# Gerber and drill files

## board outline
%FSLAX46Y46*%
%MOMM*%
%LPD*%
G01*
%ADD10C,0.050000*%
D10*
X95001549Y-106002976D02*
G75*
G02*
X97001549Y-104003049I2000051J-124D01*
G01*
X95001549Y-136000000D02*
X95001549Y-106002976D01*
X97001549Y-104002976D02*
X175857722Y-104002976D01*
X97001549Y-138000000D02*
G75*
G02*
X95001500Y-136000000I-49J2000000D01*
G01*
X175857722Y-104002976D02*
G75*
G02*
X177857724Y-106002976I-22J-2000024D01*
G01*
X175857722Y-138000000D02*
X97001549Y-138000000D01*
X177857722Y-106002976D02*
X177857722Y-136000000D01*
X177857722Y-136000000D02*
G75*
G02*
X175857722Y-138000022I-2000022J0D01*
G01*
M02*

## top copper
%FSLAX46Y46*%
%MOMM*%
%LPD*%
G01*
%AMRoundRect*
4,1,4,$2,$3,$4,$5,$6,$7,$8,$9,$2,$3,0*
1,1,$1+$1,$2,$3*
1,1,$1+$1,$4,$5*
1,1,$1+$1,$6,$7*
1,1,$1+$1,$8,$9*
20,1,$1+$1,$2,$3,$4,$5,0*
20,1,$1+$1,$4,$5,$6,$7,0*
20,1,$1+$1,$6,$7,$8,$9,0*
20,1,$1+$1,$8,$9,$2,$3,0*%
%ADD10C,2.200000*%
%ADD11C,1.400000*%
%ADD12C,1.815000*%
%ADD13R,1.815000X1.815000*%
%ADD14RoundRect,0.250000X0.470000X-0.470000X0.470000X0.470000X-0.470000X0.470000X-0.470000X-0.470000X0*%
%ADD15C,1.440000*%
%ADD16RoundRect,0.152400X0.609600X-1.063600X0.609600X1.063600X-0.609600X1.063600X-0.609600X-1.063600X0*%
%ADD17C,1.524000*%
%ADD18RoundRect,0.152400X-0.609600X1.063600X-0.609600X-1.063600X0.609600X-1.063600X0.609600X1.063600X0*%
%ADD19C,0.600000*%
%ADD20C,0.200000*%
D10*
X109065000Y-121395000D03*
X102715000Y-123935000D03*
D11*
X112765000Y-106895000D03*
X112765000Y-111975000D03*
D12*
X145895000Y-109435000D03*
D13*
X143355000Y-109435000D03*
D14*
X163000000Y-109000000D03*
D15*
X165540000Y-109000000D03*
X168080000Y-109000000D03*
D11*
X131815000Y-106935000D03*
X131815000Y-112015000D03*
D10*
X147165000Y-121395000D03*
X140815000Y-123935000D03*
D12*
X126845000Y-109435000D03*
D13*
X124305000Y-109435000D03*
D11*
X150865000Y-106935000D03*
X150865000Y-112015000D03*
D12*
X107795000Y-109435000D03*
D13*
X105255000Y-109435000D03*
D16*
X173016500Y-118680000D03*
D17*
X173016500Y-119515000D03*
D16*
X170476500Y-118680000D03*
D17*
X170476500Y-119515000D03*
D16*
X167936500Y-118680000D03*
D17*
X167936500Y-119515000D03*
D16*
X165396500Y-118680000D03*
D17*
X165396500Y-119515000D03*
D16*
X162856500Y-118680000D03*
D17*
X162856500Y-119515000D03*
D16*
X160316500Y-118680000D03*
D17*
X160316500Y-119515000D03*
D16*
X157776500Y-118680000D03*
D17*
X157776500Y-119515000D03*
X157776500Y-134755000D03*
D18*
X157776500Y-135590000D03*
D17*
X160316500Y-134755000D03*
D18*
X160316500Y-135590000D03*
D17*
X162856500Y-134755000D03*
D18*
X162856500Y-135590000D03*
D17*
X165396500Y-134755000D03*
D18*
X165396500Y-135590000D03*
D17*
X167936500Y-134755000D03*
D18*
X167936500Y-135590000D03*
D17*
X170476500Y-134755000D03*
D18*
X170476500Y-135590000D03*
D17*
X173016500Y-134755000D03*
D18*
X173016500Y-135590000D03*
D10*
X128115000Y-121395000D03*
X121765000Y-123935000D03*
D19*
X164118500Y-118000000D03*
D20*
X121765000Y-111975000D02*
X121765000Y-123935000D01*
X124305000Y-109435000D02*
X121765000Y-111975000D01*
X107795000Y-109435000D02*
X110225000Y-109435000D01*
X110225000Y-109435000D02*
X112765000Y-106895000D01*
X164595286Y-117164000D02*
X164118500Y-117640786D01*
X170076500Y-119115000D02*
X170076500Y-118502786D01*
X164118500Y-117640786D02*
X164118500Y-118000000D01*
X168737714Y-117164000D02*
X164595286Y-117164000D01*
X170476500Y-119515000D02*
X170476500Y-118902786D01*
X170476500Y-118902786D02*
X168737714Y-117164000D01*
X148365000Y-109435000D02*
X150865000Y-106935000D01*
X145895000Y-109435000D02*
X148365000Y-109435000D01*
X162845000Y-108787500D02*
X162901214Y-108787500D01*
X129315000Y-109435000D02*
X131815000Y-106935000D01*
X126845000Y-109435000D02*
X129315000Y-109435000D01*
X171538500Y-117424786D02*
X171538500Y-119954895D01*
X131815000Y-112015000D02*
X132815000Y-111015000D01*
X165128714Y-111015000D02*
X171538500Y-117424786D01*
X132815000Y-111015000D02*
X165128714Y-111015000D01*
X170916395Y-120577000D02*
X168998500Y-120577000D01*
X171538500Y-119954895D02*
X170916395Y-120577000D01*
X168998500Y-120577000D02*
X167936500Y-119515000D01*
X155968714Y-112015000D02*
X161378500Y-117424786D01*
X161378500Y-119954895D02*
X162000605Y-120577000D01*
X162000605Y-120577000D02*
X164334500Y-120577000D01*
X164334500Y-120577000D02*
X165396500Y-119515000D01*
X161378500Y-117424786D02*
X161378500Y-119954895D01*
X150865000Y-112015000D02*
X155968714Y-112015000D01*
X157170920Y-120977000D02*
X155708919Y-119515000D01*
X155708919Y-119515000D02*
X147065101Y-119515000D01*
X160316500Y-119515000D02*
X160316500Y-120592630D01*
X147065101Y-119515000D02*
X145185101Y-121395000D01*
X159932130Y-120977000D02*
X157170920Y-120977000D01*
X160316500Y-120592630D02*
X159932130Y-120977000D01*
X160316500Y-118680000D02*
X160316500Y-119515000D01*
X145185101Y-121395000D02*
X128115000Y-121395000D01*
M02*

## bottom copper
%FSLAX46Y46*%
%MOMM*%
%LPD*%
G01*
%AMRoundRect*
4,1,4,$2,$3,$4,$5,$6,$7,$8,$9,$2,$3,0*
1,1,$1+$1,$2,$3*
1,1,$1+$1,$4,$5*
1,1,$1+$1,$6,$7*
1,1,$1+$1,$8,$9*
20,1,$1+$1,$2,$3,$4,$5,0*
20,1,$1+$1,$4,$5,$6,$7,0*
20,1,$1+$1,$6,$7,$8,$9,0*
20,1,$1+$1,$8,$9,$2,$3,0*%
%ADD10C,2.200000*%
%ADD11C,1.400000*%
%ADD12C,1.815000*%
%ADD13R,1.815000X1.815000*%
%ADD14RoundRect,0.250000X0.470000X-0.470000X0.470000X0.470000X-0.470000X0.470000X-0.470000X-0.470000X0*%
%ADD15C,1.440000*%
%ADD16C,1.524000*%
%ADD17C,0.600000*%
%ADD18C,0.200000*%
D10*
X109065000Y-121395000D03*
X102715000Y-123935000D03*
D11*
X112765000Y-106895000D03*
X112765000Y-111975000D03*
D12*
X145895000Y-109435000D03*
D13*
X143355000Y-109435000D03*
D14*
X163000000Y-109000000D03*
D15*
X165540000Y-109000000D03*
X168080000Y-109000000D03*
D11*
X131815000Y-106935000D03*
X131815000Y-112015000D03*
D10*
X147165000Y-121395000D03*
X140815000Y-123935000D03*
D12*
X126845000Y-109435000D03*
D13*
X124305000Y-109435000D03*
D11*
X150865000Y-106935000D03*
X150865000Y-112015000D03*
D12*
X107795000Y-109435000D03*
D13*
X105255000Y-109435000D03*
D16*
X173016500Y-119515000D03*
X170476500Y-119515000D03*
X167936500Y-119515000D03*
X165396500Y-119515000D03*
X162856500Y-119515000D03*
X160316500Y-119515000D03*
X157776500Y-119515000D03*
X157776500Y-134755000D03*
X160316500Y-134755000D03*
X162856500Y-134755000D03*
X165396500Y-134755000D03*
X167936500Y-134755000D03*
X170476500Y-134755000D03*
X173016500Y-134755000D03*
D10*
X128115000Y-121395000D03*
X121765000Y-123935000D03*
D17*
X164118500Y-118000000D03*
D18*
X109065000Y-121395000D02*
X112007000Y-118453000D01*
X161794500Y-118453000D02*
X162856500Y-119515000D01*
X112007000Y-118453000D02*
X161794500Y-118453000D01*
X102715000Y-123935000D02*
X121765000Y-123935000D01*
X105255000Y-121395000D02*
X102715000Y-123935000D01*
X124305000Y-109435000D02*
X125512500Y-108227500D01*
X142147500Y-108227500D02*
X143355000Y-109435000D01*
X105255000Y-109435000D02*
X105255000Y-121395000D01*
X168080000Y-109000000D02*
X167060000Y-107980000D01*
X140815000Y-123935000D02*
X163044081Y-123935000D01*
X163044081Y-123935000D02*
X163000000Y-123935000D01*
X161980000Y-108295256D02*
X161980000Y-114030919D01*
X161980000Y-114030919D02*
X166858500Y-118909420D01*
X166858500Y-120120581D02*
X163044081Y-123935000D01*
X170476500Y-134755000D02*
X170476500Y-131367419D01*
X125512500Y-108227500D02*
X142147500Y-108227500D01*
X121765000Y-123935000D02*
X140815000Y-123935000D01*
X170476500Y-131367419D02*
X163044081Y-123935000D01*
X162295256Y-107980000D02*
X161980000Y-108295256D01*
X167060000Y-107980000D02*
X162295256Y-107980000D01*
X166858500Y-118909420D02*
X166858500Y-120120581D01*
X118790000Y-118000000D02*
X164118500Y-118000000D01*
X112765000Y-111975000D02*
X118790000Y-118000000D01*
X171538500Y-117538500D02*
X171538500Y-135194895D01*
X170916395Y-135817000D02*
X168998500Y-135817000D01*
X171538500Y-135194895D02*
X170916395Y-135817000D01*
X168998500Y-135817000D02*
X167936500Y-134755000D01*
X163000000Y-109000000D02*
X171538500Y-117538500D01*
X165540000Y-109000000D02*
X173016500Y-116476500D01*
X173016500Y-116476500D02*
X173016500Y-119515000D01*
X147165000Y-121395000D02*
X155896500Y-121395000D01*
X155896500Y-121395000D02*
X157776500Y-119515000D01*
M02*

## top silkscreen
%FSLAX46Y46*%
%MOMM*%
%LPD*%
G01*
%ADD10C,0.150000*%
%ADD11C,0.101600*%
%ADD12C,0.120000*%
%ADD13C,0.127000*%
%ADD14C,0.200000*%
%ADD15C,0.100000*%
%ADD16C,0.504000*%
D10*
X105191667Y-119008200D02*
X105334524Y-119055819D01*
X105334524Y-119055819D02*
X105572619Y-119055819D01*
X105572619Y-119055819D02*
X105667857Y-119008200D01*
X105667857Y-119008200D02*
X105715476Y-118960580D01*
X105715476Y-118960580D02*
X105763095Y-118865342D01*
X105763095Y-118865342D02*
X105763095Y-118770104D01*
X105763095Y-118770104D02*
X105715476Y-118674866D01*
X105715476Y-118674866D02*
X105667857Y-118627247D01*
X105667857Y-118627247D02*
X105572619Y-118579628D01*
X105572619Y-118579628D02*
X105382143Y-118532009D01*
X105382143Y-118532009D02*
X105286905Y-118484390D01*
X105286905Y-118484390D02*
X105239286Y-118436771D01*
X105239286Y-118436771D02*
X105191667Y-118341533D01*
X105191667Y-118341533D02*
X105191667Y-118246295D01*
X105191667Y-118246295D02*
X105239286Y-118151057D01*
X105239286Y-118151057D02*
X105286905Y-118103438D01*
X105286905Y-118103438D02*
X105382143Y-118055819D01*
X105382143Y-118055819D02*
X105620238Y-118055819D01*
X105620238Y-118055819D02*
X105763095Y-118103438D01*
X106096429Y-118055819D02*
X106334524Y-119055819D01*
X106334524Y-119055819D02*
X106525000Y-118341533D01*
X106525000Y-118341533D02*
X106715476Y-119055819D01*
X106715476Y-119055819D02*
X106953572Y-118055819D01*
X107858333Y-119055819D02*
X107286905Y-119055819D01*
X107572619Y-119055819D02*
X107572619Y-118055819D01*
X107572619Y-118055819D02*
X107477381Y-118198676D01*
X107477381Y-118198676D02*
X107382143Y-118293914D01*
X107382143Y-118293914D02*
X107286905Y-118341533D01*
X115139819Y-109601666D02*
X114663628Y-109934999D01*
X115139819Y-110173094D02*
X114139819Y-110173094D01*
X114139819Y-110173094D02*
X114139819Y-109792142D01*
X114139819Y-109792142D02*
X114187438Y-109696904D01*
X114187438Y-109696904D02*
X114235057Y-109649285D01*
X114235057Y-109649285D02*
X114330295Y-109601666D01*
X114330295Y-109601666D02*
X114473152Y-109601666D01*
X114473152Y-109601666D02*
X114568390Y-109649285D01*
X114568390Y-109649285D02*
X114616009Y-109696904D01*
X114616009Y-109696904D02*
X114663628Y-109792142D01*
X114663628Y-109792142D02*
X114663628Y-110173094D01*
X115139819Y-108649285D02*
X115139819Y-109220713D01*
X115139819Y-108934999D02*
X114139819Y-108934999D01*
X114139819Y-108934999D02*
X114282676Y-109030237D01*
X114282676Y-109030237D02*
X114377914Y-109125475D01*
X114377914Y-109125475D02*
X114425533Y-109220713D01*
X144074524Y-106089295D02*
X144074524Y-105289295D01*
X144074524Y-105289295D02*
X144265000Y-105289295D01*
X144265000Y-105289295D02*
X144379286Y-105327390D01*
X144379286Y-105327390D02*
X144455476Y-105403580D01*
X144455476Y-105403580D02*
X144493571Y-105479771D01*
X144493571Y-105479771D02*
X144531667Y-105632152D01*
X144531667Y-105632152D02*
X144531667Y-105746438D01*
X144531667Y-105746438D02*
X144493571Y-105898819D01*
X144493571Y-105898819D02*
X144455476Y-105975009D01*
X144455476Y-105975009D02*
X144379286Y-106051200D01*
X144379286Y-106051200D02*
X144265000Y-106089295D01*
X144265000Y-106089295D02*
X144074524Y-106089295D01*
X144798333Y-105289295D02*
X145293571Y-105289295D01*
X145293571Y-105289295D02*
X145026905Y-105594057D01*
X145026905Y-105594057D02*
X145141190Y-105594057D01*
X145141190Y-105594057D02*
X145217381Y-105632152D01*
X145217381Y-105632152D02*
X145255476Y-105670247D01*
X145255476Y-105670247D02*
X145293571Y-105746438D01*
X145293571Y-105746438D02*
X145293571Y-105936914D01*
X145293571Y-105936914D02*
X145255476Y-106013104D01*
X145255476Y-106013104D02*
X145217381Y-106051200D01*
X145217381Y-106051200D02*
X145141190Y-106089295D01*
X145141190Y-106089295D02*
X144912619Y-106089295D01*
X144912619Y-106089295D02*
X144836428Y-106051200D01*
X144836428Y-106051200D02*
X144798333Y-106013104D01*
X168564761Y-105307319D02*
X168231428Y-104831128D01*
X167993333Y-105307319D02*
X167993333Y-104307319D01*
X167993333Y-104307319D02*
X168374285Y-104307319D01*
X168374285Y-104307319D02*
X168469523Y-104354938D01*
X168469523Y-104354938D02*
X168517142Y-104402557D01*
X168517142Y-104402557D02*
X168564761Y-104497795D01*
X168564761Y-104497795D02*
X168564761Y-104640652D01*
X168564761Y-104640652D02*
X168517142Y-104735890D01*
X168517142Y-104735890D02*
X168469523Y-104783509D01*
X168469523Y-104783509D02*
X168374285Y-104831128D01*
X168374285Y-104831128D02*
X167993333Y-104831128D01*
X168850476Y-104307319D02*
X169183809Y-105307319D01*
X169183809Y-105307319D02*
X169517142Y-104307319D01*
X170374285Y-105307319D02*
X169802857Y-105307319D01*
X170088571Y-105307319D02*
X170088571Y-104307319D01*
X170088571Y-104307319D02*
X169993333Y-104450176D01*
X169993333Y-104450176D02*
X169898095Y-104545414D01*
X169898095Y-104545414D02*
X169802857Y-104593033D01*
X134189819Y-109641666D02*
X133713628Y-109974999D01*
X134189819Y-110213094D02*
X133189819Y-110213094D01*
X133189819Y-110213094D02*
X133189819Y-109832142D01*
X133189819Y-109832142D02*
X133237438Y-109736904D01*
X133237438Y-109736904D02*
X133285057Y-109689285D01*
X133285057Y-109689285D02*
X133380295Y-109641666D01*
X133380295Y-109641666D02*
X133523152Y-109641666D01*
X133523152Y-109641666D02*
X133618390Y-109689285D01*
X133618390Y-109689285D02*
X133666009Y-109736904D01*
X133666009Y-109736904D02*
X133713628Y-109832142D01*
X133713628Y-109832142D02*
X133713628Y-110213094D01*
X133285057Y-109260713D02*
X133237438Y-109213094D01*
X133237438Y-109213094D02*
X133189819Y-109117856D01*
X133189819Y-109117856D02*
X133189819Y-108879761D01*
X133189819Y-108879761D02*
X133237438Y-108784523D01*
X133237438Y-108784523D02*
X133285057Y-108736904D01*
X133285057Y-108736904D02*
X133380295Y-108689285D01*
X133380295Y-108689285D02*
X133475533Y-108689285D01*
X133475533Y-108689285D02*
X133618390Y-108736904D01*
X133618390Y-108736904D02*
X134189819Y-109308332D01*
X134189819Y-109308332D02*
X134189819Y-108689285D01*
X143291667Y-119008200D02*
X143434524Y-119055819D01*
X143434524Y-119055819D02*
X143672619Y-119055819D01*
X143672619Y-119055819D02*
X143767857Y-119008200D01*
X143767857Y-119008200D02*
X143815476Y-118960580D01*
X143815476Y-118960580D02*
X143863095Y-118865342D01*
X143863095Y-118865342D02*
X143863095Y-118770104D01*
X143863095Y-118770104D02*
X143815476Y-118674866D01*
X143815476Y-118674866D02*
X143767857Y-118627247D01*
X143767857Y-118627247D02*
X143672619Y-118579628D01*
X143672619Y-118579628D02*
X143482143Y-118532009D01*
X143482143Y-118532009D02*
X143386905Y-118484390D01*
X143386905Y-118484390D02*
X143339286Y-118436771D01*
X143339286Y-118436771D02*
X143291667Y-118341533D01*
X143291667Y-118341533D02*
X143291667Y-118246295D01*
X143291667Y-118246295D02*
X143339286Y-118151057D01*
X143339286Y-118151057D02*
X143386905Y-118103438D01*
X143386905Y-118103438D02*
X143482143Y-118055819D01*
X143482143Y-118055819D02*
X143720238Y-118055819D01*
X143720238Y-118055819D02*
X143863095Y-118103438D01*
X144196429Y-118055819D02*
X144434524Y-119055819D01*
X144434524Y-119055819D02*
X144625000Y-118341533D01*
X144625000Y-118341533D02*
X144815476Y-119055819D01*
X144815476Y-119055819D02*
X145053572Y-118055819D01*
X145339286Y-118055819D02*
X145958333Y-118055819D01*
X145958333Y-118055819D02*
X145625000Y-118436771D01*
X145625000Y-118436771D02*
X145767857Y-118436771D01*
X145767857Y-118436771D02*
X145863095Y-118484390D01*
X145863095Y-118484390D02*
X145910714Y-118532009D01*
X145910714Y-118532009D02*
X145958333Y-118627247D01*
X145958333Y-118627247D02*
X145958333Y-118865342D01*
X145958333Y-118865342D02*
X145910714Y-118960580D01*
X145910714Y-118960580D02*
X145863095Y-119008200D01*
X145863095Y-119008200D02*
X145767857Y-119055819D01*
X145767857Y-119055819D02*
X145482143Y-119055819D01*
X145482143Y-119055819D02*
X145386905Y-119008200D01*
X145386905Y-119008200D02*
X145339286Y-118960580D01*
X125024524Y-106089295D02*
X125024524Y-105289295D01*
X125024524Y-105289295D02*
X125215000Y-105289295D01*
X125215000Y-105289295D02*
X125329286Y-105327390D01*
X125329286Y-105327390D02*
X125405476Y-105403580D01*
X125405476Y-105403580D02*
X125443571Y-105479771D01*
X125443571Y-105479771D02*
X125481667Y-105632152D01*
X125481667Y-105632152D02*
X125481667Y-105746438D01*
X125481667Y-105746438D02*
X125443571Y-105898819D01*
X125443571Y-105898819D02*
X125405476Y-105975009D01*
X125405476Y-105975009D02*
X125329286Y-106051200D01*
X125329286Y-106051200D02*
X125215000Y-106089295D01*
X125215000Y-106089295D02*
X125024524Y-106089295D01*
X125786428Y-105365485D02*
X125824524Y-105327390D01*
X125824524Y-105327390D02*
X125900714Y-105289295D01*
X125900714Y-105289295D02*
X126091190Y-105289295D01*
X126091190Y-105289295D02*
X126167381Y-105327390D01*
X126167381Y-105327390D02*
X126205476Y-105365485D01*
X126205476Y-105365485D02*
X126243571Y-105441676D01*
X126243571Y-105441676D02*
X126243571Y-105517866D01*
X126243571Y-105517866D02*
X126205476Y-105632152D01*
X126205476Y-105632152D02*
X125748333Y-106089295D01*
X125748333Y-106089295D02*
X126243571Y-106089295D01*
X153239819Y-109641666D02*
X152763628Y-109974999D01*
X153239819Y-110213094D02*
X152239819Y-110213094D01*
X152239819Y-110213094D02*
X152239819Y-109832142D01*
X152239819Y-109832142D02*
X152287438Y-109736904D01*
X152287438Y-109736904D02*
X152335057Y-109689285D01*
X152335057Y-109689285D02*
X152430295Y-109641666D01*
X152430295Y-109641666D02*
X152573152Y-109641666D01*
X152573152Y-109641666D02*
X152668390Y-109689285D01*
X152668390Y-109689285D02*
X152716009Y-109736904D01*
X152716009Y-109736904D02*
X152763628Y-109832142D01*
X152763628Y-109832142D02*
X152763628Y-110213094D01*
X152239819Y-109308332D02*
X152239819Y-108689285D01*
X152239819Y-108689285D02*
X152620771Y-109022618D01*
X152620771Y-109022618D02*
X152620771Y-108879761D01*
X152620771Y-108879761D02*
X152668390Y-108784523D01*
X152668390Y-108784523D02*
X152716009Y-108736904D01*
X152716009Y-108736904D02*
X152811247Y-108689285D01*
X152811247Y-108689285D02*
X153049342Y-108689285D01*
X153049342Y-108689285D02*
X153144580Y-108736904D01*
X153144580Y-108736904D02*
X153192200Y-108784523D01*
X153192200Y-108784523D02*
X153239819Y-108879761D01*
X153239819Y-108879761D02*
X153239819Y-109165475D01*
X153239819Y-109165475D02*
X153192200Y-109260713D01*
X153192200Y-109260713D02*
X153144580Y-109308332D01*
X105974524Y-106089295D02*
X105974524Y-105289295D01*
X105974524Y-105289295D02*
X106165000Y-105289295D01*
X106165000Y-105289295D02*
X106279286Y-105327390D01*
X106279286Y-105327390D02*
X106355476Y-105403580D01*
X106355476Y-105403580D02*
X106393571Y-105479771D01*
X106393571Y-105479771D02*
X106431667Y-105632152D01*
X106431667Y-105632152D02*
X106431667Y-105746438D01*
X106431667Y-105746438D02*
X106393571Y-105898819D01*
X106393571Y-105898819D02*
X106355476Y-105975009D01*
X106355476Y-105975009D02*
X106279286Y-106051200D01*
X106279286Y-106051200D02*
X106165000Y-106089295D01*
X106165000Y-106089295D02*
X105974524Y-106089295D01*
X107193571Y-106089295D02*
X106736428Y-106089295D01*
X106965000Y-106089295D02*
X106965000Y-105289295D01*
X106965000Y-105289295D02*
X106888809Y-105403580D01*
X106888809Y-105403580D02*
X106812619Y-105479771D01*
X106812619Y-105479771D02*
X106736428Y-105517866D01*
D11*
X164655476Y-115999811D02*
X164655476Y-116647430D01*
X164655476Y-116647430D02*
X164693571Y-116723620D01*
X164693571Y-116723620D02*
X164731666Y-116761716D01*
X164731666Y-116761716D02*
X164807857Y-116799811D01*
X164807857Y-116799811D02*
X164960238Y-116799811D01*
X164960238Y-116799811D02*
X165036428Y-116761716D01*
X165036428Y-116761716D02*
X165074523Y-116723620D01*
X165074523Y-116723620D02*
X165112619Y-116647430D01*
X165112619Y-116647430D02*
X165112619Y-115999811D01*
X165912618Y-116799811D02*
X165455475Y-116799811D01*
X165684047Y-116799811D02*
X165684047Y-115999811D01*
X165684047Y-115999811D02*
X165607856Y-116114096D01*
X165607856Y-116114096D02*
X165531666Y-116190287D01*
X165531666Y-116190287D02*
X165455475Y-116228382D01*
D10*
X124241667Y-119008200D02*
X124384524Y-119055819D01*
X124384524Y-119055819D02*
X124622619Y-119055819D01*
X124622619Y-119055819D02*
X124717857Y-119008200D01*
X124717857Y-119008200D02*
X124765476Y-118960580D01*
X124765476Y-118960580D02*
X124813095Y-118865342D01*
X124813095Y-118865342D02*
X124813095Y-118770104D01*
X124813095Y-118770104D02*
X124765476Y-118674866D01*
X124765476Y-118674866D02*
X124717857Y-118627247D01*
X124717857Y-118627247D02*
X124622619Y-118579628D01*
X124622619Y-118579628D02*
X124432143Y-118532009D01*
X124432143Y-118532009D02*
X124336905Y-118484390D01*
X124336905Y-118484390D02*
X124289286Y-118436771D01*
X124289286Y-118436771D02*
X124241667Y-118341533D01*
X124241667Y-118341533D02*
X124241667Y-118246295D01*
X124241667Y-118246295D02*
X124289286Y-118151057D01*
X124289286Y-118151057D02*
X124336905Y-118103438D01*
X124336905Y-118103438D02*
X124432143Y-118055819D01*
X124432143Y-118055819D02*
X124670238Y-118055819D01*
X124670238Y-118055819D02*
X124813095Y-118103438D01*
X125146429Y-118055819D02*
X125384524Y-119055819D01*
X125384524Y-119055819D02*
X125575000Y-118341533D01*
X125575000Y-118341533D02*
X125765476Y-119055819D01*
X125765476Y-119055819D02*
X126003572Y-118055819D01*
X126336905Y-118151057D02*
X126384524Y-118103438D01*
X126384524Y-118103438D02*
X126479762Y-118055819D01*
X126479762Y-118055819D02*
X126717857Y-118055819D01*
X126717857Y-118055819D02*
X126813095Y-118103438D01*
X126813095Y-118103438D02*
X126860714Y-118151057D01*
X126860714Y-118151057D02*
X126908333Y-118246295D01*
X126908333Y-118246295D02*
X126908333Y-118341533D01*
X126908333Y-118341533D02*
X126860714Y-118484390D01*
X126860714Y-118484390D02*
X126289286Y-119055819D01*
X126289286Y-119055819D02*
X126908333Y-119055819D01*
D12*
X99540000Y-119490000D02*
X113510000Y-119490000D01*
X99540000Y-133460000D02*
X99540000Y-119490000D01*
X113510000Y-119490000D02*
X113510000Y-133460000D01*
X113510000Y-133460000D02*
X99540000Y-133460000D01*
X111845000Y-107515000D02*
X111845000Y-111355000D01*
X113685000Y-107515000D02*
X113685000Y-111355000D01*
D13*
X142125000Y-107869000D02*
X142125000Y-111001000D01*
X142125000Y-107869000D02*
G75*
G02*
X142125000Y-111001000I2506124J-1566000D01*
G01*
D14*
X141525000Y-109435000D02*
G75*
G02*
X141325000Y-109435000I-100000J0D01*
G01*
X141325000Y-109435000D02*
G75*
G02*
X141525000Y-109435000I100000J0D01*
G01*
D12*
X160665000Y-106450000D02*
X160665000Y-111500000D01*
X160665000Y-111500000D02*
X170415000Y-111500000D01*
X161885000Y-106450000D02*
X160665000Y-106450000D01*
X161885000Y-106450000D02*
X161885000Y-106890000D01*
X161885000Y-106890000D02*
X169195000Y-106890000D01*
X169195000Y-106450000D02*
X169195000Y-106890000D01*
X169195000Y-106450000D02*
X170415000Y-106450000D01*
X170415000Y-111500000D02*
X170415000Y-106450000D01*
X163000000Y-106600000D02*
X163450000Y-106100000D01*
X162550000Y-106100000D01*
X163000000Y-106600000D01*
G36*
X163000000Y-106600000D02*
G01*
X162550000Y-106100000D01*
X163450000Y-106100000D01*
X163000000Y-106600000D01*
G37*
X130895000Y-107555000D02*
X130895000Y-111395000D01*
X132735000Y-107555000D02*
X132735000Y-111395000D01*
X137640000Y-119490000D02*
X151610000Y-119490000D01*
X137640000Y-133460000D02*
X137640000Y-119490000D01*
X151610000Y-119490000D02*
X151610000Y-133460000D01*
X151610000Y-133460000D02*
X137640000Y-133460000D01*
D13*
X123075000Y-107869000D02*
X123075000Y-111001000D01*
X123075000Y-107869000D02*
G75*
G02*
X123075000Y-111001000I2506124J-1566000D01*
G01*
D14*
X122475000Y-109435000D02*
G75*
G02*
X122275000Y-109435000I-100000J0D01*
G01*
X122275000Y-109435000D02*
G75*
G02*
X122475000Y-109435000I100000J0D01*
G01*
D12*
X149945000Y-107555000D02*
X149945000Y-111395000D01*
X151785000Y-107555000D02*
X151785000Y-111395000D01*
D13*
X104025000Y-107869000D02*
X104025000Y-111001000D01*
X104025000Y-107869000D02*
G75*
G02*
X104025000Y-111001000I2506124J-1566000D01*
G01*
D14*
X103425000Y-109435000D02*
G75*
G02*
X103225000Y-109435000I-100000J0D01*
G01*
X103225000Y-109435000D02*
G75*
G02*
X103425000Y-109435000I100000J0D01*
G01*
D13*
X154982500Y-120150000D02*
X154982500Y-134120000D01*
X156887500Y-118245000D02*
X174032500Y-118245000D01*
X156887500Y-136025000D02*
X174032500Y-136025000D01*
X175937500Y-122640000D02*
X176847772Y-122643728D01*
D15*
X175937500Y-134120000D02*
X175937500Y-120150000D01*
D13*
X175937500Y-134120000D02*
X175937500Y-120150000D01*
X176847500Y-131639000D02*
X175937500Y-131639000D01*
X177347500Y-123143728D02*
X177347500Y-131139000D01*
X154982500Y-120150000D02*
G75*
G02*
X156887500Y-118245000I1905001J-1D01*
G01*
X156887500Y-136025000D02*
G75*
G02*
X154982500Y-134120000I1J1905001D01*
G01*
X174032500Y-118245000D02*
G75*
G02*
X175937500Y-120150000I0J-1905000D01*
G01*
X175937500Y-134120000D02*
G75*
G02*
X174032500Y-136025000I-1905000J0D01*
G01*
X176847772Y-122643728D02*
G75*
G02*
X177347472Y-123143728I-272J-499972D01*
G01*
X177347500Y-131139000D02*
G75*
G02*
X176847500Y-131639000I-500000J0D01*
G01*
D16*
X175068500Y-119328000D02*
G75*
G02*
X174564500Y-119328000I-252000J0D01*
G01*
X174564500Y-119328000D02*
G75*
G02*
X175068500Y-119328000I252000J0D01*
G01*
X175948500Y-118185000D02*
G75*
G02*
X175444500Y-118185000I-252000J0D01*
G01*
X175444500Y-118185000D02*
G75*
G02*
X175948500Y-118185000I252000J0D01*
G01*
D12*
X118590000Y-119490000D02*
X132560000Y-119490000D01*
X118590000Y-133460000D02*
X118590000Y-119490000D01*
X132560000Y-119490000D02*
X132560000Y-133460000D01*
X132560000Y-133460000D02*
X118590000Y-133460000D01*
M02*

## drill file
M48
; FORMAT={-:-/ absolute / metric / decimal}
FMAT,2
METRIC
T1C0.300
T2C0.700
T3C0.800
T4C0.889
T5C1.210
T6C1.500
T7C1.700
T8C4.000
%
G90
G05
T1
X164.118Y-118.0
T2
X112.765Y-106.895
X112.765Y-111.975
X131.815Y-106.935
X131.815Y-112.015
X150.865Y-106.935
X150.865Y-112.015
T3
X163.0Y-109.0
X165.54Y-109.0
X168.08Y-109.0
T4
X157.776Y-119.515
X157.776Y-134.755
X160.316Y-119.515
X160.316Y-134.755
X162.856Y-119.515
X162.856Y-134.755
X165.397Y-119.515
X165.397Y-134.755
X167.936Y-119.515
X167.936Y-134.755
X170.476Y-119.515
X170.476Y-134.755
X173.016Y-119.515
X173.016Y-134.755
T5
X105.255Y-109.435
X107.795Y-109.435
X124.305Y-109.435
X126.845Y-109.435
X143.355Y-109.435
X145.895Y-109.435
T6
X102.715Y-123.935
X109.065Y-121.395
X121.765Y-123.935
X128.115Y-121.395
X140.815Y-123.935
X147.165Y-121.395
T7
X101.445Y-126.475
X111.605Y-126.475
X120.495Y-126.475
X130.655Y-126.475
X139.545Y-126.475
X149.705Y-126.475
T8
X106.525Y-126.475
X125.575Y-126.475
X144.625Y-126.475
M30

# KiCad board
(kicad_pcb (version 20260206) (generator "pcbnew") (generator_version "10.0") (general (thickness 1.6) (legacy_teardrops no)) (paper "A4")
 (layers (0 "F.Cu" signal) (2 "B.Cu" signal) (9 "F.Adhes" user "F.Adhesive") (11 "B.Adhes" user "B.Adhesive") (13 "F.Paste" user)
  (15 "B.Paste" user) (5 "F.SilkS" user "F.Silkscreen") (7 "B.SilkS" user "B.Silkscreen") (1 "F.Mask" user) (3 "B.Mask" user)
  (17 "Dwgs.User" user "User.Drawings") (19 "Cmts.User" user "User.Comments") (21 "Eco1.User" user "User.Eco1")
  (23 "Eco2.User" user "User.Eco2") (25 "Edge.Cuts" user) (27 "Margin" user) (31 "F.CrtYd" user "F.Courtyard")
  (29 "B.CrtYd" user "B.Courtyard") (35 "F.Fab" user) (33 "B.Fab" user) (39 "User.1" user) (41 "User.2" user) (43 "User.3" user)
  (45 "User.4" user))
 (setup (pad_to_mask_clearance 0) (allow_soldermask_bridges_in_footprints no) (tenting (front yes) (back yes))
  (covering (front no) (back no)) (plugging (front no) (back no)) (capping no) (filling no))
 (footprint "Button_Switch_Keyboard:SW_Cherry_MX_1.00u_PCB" (layer "F.Cu") (at 109.065 121.395)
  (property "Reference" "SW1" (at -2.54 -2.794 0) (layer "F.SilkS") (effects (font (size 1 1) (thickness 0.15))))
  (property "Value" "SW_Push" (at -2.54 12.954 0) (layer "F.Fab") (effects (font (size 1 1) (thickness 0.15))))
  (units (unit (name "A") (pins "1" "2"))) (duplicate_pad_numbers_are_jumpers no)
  (fp_line (start -9.525 -1.905) (end 4.445 -1.905) (stroke (width 0.12) (type solid)) (layer "F.SilkS"))
  (fp_line (start -9.525 12.065) (end -9.525 -1.905) (stroke (width 0.12) (type solid)) (layer "F.SilkS"))
  (fp_line (start 4.445 -1.905) (end 4.445 12.065) (stroke (width 0.12) (type solid)) (layer "F.SilkS"))
  (fp_line (start 4.445 12.065) (end -9.525 12.065) (stroke (width 0.12) (type solid)) (layer "F.SilkS"))
  (pad "" np_thru_hole circle (at -7.62 5.08) (size 1.7 1.7) (drill 1.7) (layers "*.Cu" "*.Mask"))
  (pad "" np_thru_hole circle (at -2.54 5.08) (size 4 4) (drill 4) (layers "*.Cu" "*.Mask"))
  (pad "" np_thru_hole circle (at 2.54 5.08) (size 1.7 1.7) (drill 1.7) (layers "*.Cu" "*.Mask"))
  (pad "1" thru_hole circle (at 0 0) (size 2.2 2.2) (drill 1.5) (layers "*.Cu" "*.Mask") (remove_unused_layers no) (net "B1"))
  (pad "2" thru_hole circle (at -6.35 2.54) (size 2.2 2.2) (drill 1.5) (layers "*.Cu" "*.Mask") (remove_unused_layers no) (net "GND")))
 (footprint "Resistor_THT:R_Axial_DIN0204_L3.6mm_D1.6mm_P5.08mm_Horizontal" (layer "F.Cu") (at 112.765 106.895 -90)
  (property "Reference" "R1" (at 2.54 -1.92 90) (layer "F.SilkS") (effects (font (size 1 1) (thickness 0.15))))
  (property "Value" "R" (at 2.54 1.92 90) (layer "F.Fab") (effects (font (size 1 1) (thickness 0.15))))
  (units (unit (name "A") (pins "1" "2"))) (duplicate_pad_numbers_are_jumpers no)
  (fp_line (start 0.62 0.92) (end 4.46 0.92) (stroke (width 0.12) (type solid)) (layer "F.SilkS"))
  (fp_line (start 0.62 -0.92) (end 4.46 -0.92) (stroke (width 0.12) (type solid)) (layer "F.SilkS"))
  (pad "1" thru_hole circle (at 0 0 270) (size 1.4 1.4) (drill 0.7) (layers "*.Cu" "*.Mask") (remove_unused_layers no) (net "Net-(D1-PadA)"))
  (pad "2" thru_hole circle (at 5.08 0 270) (size 1.4 1.4) (drill 0.7) (layers "*.Cu" "*.Mask") (remove_unused_layers no) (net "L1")))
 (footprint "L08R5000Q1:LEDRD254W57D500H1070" (layer "F.Cu") (at 144.625 109.435)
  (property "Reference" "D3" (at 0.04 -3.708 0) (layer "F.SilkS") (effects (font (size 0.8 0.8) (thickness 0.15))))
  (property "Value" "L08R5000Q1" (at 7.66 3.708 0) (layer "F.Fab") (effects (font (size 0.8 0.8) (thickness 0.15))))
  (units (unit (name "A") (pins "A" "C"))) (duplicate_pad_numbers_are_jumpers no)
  (fp_line (start -2.5 -1.566) (end -2.5 1.566) (stroke (width 0.127) (type solid)) (layer "F.SilkS"))
  (fp_arc (start -2.5 -1.566) (mid 2.961291 0) (end -2.5 1.566) (stroke (width 0.127) (type solid)) (layer "F.SilkS"))
  (fp_circle (center -3.2 0) (end -3.1 0) (stroke (width 0.2) (type solid)) (fill no) (layer "F.SilkS"))
  (pad "A" thru_hole circle (at 1.27 0) (size 1.815 1.815) (drill 1.21) (layers "*.Cu" "*.Mask") (remove_unused_layers no)
   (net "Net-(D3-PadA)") (solder_mask_margin 0.102))
  (pad "C" thru_hole rect (at -1.27 0) (size 1.815 1.815) (drill 1.21) (layers "*.Cu" "*.Mask") (remove_unused_layers no) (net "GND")
   (solder_mask_margin 0.102)))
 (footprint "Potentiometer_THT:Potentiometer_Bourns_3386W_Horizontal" (layer "F.Cu") (at 163 109)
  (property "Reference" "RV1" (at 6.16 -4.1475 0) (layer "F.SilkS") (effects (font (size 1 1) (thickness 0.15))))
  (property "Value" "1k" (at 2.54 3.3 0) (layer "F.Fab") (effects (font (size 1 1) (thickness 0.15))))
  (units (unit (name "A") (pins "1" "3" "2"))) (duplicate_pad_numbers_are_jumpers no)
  (fp_line (start -2.335 -2.55) (end -2.335 2.5) (stroke (width 0.12) (type default)) (layer "F.SilkS"))
  (fp_line (start -2.335 2.5) (end 7.415 2.5) (stroke (width 0.12) (type default)) (layer "F.SilkS"))
  (fp_line (start -1.115 -2.55) (end -2.335 -2.55) (stroke (width 0.12) (type default)) (layer "F.SilkS"))
  (fp_line (start -1.115 -2.55) (end -1.115 -2.11) (stroke (width 0.12) (type default)) (layer "F.SilkS"))
  (fp_line (start -1.115 -2.11) (end 6.195 -2.11) (stroke (width 0.12) (type default)) (layer "F.SilkS"))
  (fp_line (start 6.195 -2.55) (end 6.195 -2.11) (stroke (width 0.12) (type default)) (layer "F.SilkS"))
  (fp_line (start 6.195 -2.55) (end 7.415 -2.55) (stroke (width 0.12) (type default)) (layer "F.SilkS"))
  (fp_line (start 7.415 2.5) (end 7.415 -2.55) (stroke (width 0.12) (type default)) (layer "F.SilkS"))
  (fp_poly (pts (xy 0 -2.4) (xy 0.45 -2.9) (xy -0.45 -2.9)) (stroke (width 0.12) (type solid)) (fill yes) (layer "F.SilkS"))
  (pad "1" thru_hole roundrect (at 0 0 90) (size 1.44 1.44) (drill 0.8) (layers "*.Cu" "*.Mask") (remove_unused_layers no)
   (roundrect_rratio 0.1736111111) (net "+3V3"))
  (pad "2" thru_hole circle (at 2.54 0 90) (size 1.44 1.44) (drill 0.8) (layers "*.Cu" "*.Mask") (remove_unused_layers no) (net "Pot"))
  (pad "3" thru_hole circle (at 5.08 0 90) (size 1.44 1.44) (drill 0.8) (layers "*.Cu" "*.Mask") (remove_unused_layers no) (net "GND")))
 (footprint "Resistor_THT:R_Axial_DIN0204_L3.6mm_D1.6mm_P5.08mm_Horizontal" (layer "F.Cu") (at 131.815 106.935 -90)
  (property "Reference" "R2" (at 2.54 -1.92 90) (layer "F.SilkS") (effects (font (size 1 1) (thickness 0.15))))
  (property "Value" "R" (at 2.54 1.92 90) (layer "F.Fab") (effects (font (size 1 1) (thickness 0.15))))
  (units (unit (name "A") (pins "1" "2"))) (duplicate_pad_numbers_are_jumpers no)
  (fp_line (start 0.62 0.92) (end 4.46 0.92) (stroke (width 0.12) (type solid)) (layer "F.SilkS"))
  (fp_line (start 0.62 -0.92) (end 4.46 -0.92) (stroke (width 0.12) (type solid)) (layer "F.SilkS"))
  (pad "1" thru_hole circle (at 0 0 270) (size 1.4 1.4) (drill 0.7) (layers "*.Cu" "*.Mask") (remove_unused_layers no) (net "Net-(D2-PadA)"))
  (pad "2" thru_hole circle (at 5.08 0 270) (size 1.4 1.4) (drill 0.7) (layers "*.Cu" "*.Mask") (remove_unused_layers no) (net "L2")))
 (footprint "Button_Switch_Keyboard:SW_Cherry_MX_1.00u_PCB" (layer "F.Cu") (at 147.165 121.395)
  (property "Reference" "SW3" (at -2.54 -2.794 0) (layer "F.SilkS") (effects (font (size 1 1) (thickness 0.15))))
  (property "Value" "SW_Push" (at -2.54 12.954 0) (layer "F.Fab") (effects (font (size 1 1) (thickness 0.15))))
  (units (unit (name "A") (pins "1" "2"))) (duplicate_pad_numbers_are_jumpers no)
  (fp_line (start -9.525 -1.905) (end 4.445 -1.905) (stroke (width 0.12) (type solid)) (layer "F.SilkS"))
  (fp_line (start -9.525 12.065) (end -9.525 -1.905) (stroke (width 0.12) (type solid)) (layer "F.SilkS"))
  (fp_line (start 4.445 -1.905) (end 4.445 12.065) (stroke (width 0.12) (type solid)) (layer "F.SilkS"))
  (fp_line (start 4.445 12.065) (end -9.525 12.065) (stroke (width 0.12) (type solid)) (layer "F.SilkS"))
  (pad "" np_thru_hole circle (at -7.62 5.08) (size 1.7 1.7) (drill 1.7) (layers "*.Cu" "*.Mask"))
  (pad "" np_thru_hole circle (at -2.54 5.08) (size 4 4) (drill 4) (layers "*.Cu" "*.Mask"))
  (pad "" np_thru_hole circle (at 2.54 5.08) (size 1.7 1.7) (drill 1.7) (layers "*.Cu" "*.Mask"))
  (pad "1" thru_hole circle (at 0 0) (size 2.2 2.2) (drill 1.5) (layers "*.Cu" "*.Mask") (remove_unused_layers no) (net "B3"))
  (pad "2" thru_hole circle (at -6.35 2.54) (size 2.2 2.2) (drill 1.5) (layers "*.Cu" "*.Mask") (remove_unused_layers no) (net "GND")))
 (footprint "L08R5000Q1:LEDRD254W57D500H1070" (layer "F.Cu") (at 125.575 109.435)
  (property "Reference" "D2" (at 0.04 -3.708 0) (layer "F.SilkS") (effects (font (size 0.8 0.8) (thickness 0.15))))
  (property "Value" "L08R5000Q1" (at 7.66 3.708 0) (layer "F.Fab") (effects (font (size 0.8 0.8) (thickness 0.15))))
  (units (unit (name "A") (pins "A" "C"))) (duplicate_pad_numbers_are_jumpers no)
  (fp_line (start -2.5 -1.566) (end -2.5 1.566) (stroke (width 0.127) (type solid)) (layer "F.SilkS"))
  (fp_arc (start -2.5 -1.566) (mid 2.961291 0) (end -2.5 1.566) (stroke (width 0.127) (type solid)) (layer "F.SilkS"))
  (fp_circle (center -3.2 0) (end -3.1 0) (stroke (width 0.2) (type solid)) (fill no) (layer "F.SilkS"))
  (pad "A" thru_hole circle (at 1.27 0) (size 1.815 1.815) (drill 1.21) (layers "*.Cu" "*.Mask") (remove_unused_layers no)
   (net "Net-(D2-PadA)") (solder_mask_margin 0.102))
  (pad "C" thru_hole rect (at -1.27 0) (size 1.815 1.815) (drill 1.21) (layers "*.Cu" "*.Mask") (remove_unused_layers no) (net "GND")
   (solder_mask_margin 0.102)))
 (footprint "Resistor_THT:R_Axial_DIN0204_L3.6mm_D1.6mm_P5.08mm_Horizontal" (layer "F.Cu") (at 150.865 106.935 -90)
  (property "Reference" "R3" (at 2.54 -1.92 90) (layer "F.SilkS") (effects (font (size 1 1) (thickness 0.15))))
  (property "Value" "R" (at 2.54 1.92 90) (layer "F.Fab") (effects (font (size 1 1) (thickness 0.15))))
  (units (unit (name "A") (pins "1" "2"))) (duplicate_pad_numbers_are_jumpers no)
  (fp_line (start 0.62 0.92) (end 4.46 0.92) (stroke (width 0.12) (type solid)) (layer "F.SilkS"))
  (fp_line (start 0.62 -0.92) (end 4.46 -0.92) (stroke (width 0.12) (type solid)) (layer "F.SilkS"))
  (pad "1" thru_hole circle (at 0 0 270) (size 1.4 1.4) (drill 0.7) (layers "*.Cu" "*.Mask") (remove_unused_layers no) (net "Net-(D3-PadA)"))
  (pad "2" thru_hole circle (at 5.08 0 270) (size 1.4 1.4) (drill 0.7) (layers "*.Cu" "*.Mask") (remove_unused_layers no) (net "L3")))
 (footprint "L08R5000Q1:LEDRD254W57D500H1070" (layer "F.Cu") (at 106.525 109.435)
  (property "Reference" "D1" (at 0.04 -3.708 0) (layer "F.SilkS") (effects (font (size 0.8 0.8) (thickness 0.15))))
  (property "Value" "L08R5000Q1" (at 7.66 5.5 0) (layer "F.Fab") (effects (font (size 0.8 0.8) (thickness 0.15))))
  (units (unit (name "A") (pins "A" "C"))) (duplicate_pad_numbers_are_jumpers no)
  (fp_line (start -2.5 -1.566) (end -2.5 1.566) (stroke (width 0.127) (type solid)) (layer "F.SilkS"))
  (fp_arc (start -2.5 -1.566) (mid 2.961291 0) (end -2.5 1.566) (stroke (width 0.127) (type solid)) (layer "F.SilkS"))
  (fp_circle (center -3.2 0) (end -3.1 0) (stroke (width 0.2) (type solid)) (fill no) (layer "F.SilkS"))
  (pad "A" thru_hole circle (at 1.27 0) (size 1.815 1.815) (drill 1.21) (layers "*.Cu" "*.Mask") (remove_unused_layers no)
   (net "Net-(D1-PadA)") (solder_mask_margin 0.102))
  (pad "C" thru_hole rect (at -1.27 0) (size 1.815 1.815) (drill 1.21) (layers "*.Cu" "*.Mask") (remove_unused_layers no) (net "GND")
   (solder_mask_margin 0.102)))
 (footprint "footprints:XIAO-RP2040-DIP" (layer "F.Cu") (at 165.3965 127.135)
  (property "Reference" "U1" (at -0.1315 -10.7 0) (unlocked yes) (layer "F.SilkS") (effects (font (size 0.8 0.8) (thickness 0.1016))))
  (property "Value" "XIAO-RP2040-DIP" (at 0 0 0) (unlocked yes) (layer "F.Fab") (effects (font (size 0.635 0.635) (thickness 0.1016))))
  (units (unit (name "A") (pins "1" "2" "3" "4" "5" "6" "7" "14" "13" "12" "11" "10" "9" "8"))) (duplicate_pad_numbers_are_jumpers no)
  (fp_line (start -10.414 -6.985) (end -10.414 6.985) (stroke (width 0.127) (type solid)) (layer "F.SilkS"))
  (fp_line (start -8.509 -8.89) (end 8.636 -8.89) (stroke (width 0.127) (type solid)) (layer "F.SilkS"))
  (fp_line (start -8.509 8.89) (end 8.636 8.89) (stroke (width 0.127) (type solid)) (layer "F.SilkS"))
  (fp_line (start 10.541 -4.495) (end 11.451272 -4.491272) (stroke (width 0.127) (type solid)) (layer "F.SilkS"))
  (fp_line (start 10.541 6.985) (end 10.541 -6.985) (stroke (width 0.1) (type solid)) (layer "F.SilkS"))
  (fp_line (start 10.541 6.985) (end 10.541 -6.985) (stroke (width 0.127) (type solid)) (layer "F.SilkS"))
  (fp_line (start 11.451 4.504) (end 10.541 4.504) (stroke (width 0.127) (type solid)) (layer "F.SilkS"))
  (fp_line (start 11.951 -3.991272) (end 11.951 4.004) (stroke (width 0.127) (type solid)) (layer "F.SilkS"))
  (fp_arc (start -10.414 -6.985) (mid -9.856038 -8.332038) (end -8.509 -8.89) (stroke (width 0.127) (type solid)) (layer "F.SilkS"))
  (fp_arc (start -8.509 8.89) (mid -9.856038 8.332038) (end -10.414 6.985) (stroke (width 0.127) (type solid)) (layer "F.SilkS"))
  (fp_arc (start 8.636 -8.89) (mid 9.983038 -8.332038) (end 10.541 -6.985) (stroke (width 0.127) (type solid)) (layer "F.SilkS"))
  (fp_arc (start 10.541 6.985) (mid 9.983038 8.332038) (end 8.636 8.89) (stroke (width 0.127) (type solid)) (layer "F.SilkS"))
  (fp_arc (start 11.451272 -4.491272) (mid 11.804644 -4.344724) (end 11.951 -3.991272) (stroke (width 0.127) (type default))
   (layer "F.SilkS"))
  (fp_arc (start 11.951 4.004) (mid 11.804553 4.357553) (end 11.451 4.504) (stroke (width 0.127) (type default)) (layer "F.SilkS"))
  (fp_circle (center 9.42 -7.807) (end 9.674 -7.807) (stroke (width 0.5) (type solid)) (fill yes) (layer "F.SilkS"))
  (fp_circle (center 10.3 -8.95) (end 10.554 -8.95) (stroke (width 0.5) (type solid)) (fill yes) (layer "F.SilkS"))
  (pad "1" smd roundrect (at 7.62 -8.455 90) (size 2.432 1.524) (layers "F.Cu" "F.Mask") (roundrect_rratio 0.1) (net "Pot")
   (thermal_bridge_angle 45))
  (pad "1" thru_hole circle (at 7.62 -7.62 90) (size 1.524 1.524) (drill 0.889) (layers "*.Cu" "*.Mask") (remove_unused_layers no)
   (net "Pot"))
  (pad "2" smd roundrect (at 5.08 -8.455 90) (size 2.432 1.524) (layers "F.Cu" "F.Mask") (roundrect_rratio 0.1) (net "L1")
   (thermal_bridge_angle 45))
  (pad "2" thru_hole circle (at 5.08 -7.62 90) (size 1.524 1.524) (drill 0.889) (layers "*.Cu" "*.Mask") (remove_unused_layers no)
   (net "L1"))
  (pad "3" smd roundrect (at 2.54 -8.455 90) (size 2.432 1.524) (layers "F.Cu" "F.Mask") (roundrect_rratio 0.1) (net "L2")
   (thermal_bridge_angle 45))
  (pad "3" thru_hole circle (at 2.54 -7.62 90) (size 1.524 1.524) (drill 0.889) (layers "*.Cu" "*.Mask") (remove_unused_layers no)
   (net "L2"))
  (pad "4" smd roundrect (at 0 -8.455 90) (size 2.432 1.524) (layers "F.Cu" "F.Mask") (roundrect_rratio 0.1) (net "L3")
   (thermal_bridge_angle 45))
  (pad "4" thru_hole circle (at 0 -7.62 90) (size 1.524 1.524) (drill 0.889) (layers "*.Cu" "*.Mask") (remove_unused_layers no) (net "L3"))
  (pad "5" smd roundrect (at -2.54 -8.455 90) (size 2.432 1.524) (layers "F.Cu" "F.Mask") (roundrect_rratio 0.1) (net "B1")
   (thermal_bridge_angle 45))
  (pad "5" thru_hole circle (at -2.54 -7.62 90) (size 1.524 1.524) (drill 0.889) (layers "*.Cu" "*.Mask") (remove_unused_layers no)
   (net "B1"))
  (pad "6" smd roundrect (at -5.08 -8.455 90) (size 2.432 1.524) (layers "F.Cu" "F.Mask") (roundrect_rratio 0.1) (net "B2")
   (thermal_bridge_angle 45))
  (pad "6" thru_hole circle (at -5.08 -7.62 90) (size 1.524 1.524) (drill 0.889) (layers "*.Cu" "*.Mask") (remove_unused_layers no)
   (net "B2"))
  (pad "7" smd roundrect (at -7.62 -8.455 90) (size 2.432 1.524) (layers "F.Cu" "F.Mask") (roundrect_rratio 0.1) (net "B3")
   (thermal_bridge_angle 45))
  (pad "7" thru_hole circle (at -7.62 -7.62 90) (size 1.524 1.524) (drill 0.889) (layers "*.Cu" "*.Mask") (remove_unused_layers no)
   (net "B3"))
  (pad "8" thru_hole circle (at -7.62 7.62 270) (size 1.524 1.524) (drill 0.889) (layers "*.Cu" "*.Mask") (remove_unused_layers no)
   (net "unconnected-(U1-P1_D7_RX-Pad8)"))
  (pad "8" smd roundrect (at -7.62 8.455 270) (size 2.432 1.524) (layers "F.Cu" "F.Mask") (roundrect_rratio 0.1)
   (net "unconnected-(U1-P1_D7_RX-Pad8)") (thermal_bridge_angle 45))
  (pad "9" thru_hole circle (at -5.08 7.62 270) (size 1.524 1.524) (drill 0.889) (layers "*.Cu" "*.Mask") (remove_unused_layers no)
   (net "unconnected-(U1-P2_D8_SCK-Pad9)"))
  (pad "9" smd roundrect (at -5.08 8.455 270) (size 2.432 1.524) (layers "F.Cu" "F.Mask") (roundrect_rratio 0.1)
   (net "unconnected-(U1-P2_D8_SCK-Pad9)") (thermal_bridge_angle 45))
  (pad "10" thru_hole circle (at -2.54 7.62 270) (size 1.524 1.524) (drill 0.889) (layers "*.Cu" "*.Mask") (remove_unused_layers no)
   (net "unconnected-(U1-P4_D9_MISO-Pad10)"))
  (pad "10" smd roundrect (at -2.54 8.455 270) (size 2.432 1.524) (layers "F.Cu" "F.Mask") (roundrect_rratio 0.1)
   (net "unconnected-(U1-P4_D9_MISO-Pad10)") (thermal_bridge_angle 45))
  (pad "11" thru_hole circle (at 0 7.62 270) (size 1.524 1.524) (drill 0.889) (layers "*.Cu" "*.Mask") (remove_unused_layers no)
   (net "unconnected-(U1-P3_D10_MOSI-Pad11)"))
  (pad "11" smd roundrect (at 0 8.455 270) (size 2.432 1.524) (layers "F.Cu" "F.Mask") (roundrect_rratio 0.1)
   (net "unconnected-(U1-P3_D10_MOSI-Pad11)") (thermal_bridge_angle 45))
  (pad "12" thru_hole circle (at 2.54 7.62 270) (size 1.524 1.524) (drill 0.889) (layers "*.Cu" "*.Mask") (remove_unused_layers no)
   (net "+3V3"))
  (pad "12" smd roundrect (at 2.54 8.455 270) (size 2.432 1.524) (layers "F.Cu" "F.Mask") (roundrect_rratio 0.1) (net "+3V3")
   (thermal_bridge_angle 45))
  (pad "13" thru_hole circle (at 5.08 7.62 270) (size 1.524 1.524) (drill 0.889) (layers "*.Cu" "*.Mask") (remove_unused_layers no)
   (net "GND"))
  (pad "13" smd roundrect (at 5.08 8.455 270) (size 2.432 1.524) (layers "F.Cu" "F.Mask") (roundrect_rratio 0.1) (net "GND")
   (thermal_bridge_angle 45))
  (pad "14" thru_hole circle (at 7.62 7.62 270) (size 1.524 1.524) (drill 0.889) (layers "*.Cu" "*.Mask") (remove_unused_layers no)
   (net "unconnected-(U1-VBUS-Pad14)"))
  (pad "14" smd roundrect (at 7.62 8.455 270) (size 2.432 1.524) (layers "F.Cu" "F.Mask") (roundrect_rratio 0.1)
   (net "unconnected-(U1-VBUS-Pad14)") (thermal_bridge_angle 45)))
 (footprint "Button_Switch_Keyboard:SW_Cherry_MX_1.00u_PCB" (layer "F.Cu") (at 128.115 121.395)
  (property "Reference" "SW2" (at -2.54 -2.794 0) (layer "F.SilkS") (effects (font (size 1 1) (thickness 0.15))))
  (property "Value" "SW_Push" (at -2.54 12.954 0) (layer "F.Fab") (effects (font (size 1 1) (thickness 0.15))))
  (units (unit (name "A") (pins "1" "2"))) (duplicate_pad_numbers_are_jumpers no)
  (fp_line (start -9.525 -1.905) (end 4.445 -1.905) (stroke (width 0.12) (type solid)) (layer "F.SilkS"))
  (fp_line (start -9.525 12.065) (end -9.525 -1.905) (stroke (width 0.12) (type solid)) (layer "F.SilkS"))
  (fp_line (start 4.445 -1.905) (end 4.445 12.065) (stroke (width 0.12) (type solid)) (layer "F.SilkS"))
  (fp_line (start 4.445 12.065) (end -9.525 12.065) (stroke (width 0.12) (type solid)) (layer "F.SilkS"))
  (pad "" np_thru_hole circle (at -7.62 5.08) (size 1.7 1.7) (drill 1.7) (layers "*.Cu" "*.Mask"))
  (pad "" np_thru_hole circle (at -2.54 5.08) (size 4 4) (drill 4) (layers "*.Cu" "*.Mask"))
  (pad "" np_thru_hole circle (at 2.54 5.08) (size 1.7 1.7) (drill 1.7) (layers "*.Cu" "*.Mask"))
  (pad "1" thru_hole circle (at 0 0) (size 2.2 2.2) (drill 1.5) (layers "*.Cu" "*.Mask") (remove_unused_layers no) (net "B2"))
  (pad "2" thru_hole circle (at -6.35 2.54) (size 2.2 2.2) (drill 1.5) (layers "*.Cu" "*.Mask") (remove_unused_layers no) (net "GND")))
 (gr_arc (start 95.001549 106.002976) (mid 95.587347 104.588795) (end 97.001549 104.002976) (stroke (width 0.05) (type default))
  (layer "Edge.Cuts"))
 (gr_line (start 95.001549 136) (end 95.001549 106.002976) (stroke (width 0.05) (type default)) (layer "Edge.Cuts"))
 (gr_line (start 97.001549 104.002976) (end 175.857722 104.002976) (stroke (width 0.05) (type default)) (layer "Edge.Cuts"))
 (gr_arc (start 97.001549 138) (mid 95.587335 137.414214) (end 95.001549 136) (stroke (width 0.05) (type default)) (layer "Edge.Cuts"))
 (gr_arc (start 175.857722 104.002976) (mid 177.271936 104.588762) (end 177.857722 106.002976) (stroke (width 0.05) (type default))
  (layer "Edge.Cuts"))
 (gr_line (start 175.857722 138) (end 97.001549 138) (stroke (width 0.05) (type default)) (layer "Edge.Cuts"))
 (gr_line (start 177.857722 106.002976) (end 177.857722 136) (stroke (width 0.05) (type default)) (layer "Edge.Cuts"))
 (gr_arc (start 177.857722 136) (mid 177.271937 137.414221) (end 175.857722 138) (stroke (width 0.05) (type default)) (layer "Edge.Cuts"))
 (segment (start 109.065 121.395) (end 112.007 118.453) (width 0.2) (layer "B.Cu") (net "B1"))
 (segment (start 161.7945 118.453) (end 162.8565 119.515) (width 0.2) (layer "B.Cu") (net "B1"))
 (segment (start 112.007 118.453) (end 161.7945 118.453) (width 0.2) (layer "B.Cu") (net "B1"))
 (segment (start 121.765 111.975) (end 121.765 123.935) (width 0.2) (layer "F.Cu") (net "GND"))
 (segment (start 124.305 109.435) (end 121.765 111.975) (width 0.2) (layer "F.Cu") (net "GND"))
 (segment (start 102.715 123.935) (end 121.765 123.935) (width 0.2) (layer "B.Cu") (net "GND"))
 (segment (start 105.255 121.395) (end 102.715 123.935) (width 0.2) (layer "B.Cu") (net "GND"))
 (segment (start 124.305 109.435) (end 125.5125 108.2275) (width 0.2) (layer "B.Cu") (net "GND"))
 (segment (start 142.1475 108.2275) (end 143.355 109.435) (width 0.2) (layer "B.Cu") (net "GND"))
 (segment (start 105.255 109.435) (end 105.255 121.395) (width 0.2) (layer "B.Cu") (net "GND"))
 (segment (start 168.08 109) (end 167.06 107.98) (width 0.2) (layer "B.Cu") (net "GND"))
 (segment (start 140.815 123.935) (end 163.044081 123.935) (width 0.2) (layer "B.Cu") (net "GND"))
 (segment (start 163.044081 123.935) (end 163 123.935) (width 0.2) (layer "B.Cu") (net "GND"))
 (segment (start 161.98 108.295256) (end 161.98 114.030919) (width 0.2) (layer "B.Cu") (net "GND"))
 (segment (start 161.98 114.030919) (end 166.8585 118.90942) (width 0.2) (layer "B.Cu") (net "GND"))
 (segment (start 166.8585 120.120581) (end 163.044081 123.935) (width 0.2) (layer "B.Cu") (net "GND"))
 (segment (start 170.4765 134.755) (end 170.4765 131.367419) (width 0.2) (layer "B.Cu") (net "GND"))
 (segment (start 125.5125 108.2275) (end 142.1475 108.2275) (width 0.2) (layer "B.Cu") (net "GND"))
 (segment (start 121.765 123.935) (end 140.815 123.935) (width 0.2) (layer "B.Cu") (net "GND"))
 (segment (start 170.4765 131.367419) (end 163.044081 123.935) (width 0.2) (layer "B.Cu") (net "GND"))
 (segment (start 162.295256 107.98) (end 161.98 108.295256) (width 0.2) (layer "B.Cu") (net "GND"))
 (segment (start 167.06 107.98) (end 162.295256 107.98) (width 0.2) (layer "B.Cu") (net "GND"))
 (segment (start 166.8585 118.90942) (end 166.8585 120.120581) (width 0.2) (layer "B.Cu") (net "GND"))
 (segment (start 107.795 109.435) (end 110.225 109.435) (width 0.2) (layer "F.Cu") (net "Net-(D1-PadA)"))
 (segment (start 110.225 109.435) (end 112.765 106.895) (width 0.2) (layer "F.Cu") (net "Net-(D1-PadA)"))
 (segment (start 164.595286 117.164) (end 164.1185 117.640786) (width 0.2) (layer "F.Cu") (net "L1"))
 (segment (start 170.0765 119.115) (end 170.0765 118.502786) (width 0.2) (layer "F.Cu") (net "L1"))
 (segment (start 164.1185 117.640786) (end 164.1185 118) (width 0.2) (layer "F.Cu") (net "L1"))
 (segment (start 168.737714 117.164) (end 164.595286 117.164) (width 0.2) (layer "F.Cu") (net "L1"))
 (segment (start 170.4765 119.515) (end 170.4765 118.902786) (width 0.2) (layer "F.Cu") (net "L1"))
 (segment (start 170.4765 118.902786) (end 168.737714 117.164) (width 0.2) (layer "F.Cu") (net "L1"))
 (via (at 164.1185 118) (size 0.6) (drill 0.3) (layers "F.Cu" "B.Cu") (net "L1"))
 (segment (start 118.79 118) (end 164.1185 118) (width 0.2) (layer "B.Cu") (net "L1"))
 (segment (start 112.765 111.975) (end 118.79 118) (width 0.2) (layer "B.Cu") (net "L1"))
 (segment (start 148.365 109.435) (end 150.865 106.935) (width 0.2) (layer "F.Cu") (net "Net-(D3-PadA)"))
 (segment (start 145.895 109.435) (end 148.365 109.435) (width 0.2) (layer "F.Cu") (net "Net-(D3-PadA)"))
 (segment (start 162.845 108.7875) (end 162.901214 108.7875) (width 0.2) (layer "F.Cu") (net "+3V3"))
 (segment (start 171.5385 117.5385) (end 171.5385 135.194895) (width 0.2) (layer "B.Cu") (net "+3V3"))
 (segment (start 170.916395 135.817) (end 168.9985 135.817) (width 0.2) (layer "B.Cu") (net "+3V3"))
 (segment (start 171.5385 135.194895) (end 170.916395 135.817) (width 0.2) (layer "B.Cu") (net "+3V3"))
 (segment (start 168.9985 135.817) (end 167.9365 134.755) (width 0.2) (layer "B.Cu") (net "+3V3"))
 (segment (start 163 109) (end 171.5385 117.5385) (width 0.2) (layer "B.Cu") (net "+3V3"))
 (segment (start 165.54 109) (end 173.0165 116.4765) (width 0.2) (layer "B.Cu") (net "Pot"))
 (segment (start 173.0165 116.4765) (end 173.0165 119.515) (width 0.2) (layer "B.Cu") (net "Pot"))
 (segment (start 129.315 109.435) (end 131.815 106.935) (width 0.2) (layer "F.Cu") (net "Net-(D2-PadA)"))
 (segment (start 126.845 109.435) (end 129.315 109.435) (width 0.2) (layer "F.Cu") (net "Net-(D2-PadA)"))
 (segment (start 171.5385 117.424786) (end 171.5385 119.954895) (width 0.2) (layer "F.Cu") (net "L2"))
 (segment (start 131.815 112.015) (end 132.815 111.015) (width 0.2) (layer "F.Cu") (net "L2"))
 (segment (start 165.128714 111.015) (end 171.5385 117.424786) (width 0.2) (layer "F.Cu") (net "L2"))
 (segment (start 132.815 111.015) (end 165.128714 111.015) (width 0.2) (layer "F.Cu") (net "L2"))
 (segment (start 170.916395 120.577) (end 168.9985 120.577) (width 0.2) (layer "F.Cu") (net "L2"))
 (segment (start 171.5385 119.954895) (end 170.916395 120.577) (width 0.2) (layer "F.Cu") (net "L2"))
 (segment (start 168.9985 120.577) (end 167.9365 119.515) (width 0.2) (layer "F.Cu") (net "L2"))
 (segment (start 147.165 121.395) (end 155.8965 121.395) (width 0.2) (layer "B.Cu") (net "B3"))
 (segment (start 155.8965 121.395) (end 157.7765 119.515) (width 0.2) (layer "B.Cu") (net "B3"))
 (segment (start 155.968714 112.015) (end 161.3785 117.424786) (width 0.2) (layer "F.Cu") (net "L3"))
 (segment (start 161.3785 119.954895) (end 162.000605 120.577) (width 0.2) (layer "F.Cu") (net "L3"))
 (segment (start 162.000605 120.577) (end 164.3345 120.577) (width 0.2) (layer "F.Cu") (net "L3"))
 (segment (start 164.3345 120.577) (end 165.3965 119.515) (width 0.2) (layer "F.Cu") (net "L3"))
 (segment (start 161.3785 117.424786) (end 161.3785 119.954895) (width 0.2) (layer "F.Cu") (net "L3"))
 (segment (start 150.865 112.015) (end 155.968714 112.015) (width 0.2) (layer "F.Cu") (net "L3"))
 (segment (start 157.17092 120.977) (end 155.708919 119.515) (width 0.2) (layer "F.Cu") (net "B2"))
 (segment (start 155.708919 119.515) (end 147.065101 119.515) (width 0.2) (layer "F.Cu") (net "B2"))
 (segment (start 160.3165 119.515) (end 160.3165 120.59263) (width 0.2) (layer "F.Cu") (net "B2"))
 (segment (start 147.065101 119.515) (end 145.185101 121.395) (width 0.2) (layer "F.Cu") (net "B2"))
 (segment (start 159.93213 120.977) (end 157.17092 120.977) (width 0.2) (layer "F.Cu") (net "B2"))
 (segment (start 160.3165 120.59263) (end 159.93213 120.977) (width 0.2) (layer "F.Cu") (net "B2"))
 (segment (start 160.3165 118.68) (end 160.3165 119.515) (width 0.2) (layer "F.Cu") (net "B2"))
 (segment (start 145.185101 121.395) (end 128.115 121.395) (width 0.2) (layer "F.Cu") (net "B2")))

